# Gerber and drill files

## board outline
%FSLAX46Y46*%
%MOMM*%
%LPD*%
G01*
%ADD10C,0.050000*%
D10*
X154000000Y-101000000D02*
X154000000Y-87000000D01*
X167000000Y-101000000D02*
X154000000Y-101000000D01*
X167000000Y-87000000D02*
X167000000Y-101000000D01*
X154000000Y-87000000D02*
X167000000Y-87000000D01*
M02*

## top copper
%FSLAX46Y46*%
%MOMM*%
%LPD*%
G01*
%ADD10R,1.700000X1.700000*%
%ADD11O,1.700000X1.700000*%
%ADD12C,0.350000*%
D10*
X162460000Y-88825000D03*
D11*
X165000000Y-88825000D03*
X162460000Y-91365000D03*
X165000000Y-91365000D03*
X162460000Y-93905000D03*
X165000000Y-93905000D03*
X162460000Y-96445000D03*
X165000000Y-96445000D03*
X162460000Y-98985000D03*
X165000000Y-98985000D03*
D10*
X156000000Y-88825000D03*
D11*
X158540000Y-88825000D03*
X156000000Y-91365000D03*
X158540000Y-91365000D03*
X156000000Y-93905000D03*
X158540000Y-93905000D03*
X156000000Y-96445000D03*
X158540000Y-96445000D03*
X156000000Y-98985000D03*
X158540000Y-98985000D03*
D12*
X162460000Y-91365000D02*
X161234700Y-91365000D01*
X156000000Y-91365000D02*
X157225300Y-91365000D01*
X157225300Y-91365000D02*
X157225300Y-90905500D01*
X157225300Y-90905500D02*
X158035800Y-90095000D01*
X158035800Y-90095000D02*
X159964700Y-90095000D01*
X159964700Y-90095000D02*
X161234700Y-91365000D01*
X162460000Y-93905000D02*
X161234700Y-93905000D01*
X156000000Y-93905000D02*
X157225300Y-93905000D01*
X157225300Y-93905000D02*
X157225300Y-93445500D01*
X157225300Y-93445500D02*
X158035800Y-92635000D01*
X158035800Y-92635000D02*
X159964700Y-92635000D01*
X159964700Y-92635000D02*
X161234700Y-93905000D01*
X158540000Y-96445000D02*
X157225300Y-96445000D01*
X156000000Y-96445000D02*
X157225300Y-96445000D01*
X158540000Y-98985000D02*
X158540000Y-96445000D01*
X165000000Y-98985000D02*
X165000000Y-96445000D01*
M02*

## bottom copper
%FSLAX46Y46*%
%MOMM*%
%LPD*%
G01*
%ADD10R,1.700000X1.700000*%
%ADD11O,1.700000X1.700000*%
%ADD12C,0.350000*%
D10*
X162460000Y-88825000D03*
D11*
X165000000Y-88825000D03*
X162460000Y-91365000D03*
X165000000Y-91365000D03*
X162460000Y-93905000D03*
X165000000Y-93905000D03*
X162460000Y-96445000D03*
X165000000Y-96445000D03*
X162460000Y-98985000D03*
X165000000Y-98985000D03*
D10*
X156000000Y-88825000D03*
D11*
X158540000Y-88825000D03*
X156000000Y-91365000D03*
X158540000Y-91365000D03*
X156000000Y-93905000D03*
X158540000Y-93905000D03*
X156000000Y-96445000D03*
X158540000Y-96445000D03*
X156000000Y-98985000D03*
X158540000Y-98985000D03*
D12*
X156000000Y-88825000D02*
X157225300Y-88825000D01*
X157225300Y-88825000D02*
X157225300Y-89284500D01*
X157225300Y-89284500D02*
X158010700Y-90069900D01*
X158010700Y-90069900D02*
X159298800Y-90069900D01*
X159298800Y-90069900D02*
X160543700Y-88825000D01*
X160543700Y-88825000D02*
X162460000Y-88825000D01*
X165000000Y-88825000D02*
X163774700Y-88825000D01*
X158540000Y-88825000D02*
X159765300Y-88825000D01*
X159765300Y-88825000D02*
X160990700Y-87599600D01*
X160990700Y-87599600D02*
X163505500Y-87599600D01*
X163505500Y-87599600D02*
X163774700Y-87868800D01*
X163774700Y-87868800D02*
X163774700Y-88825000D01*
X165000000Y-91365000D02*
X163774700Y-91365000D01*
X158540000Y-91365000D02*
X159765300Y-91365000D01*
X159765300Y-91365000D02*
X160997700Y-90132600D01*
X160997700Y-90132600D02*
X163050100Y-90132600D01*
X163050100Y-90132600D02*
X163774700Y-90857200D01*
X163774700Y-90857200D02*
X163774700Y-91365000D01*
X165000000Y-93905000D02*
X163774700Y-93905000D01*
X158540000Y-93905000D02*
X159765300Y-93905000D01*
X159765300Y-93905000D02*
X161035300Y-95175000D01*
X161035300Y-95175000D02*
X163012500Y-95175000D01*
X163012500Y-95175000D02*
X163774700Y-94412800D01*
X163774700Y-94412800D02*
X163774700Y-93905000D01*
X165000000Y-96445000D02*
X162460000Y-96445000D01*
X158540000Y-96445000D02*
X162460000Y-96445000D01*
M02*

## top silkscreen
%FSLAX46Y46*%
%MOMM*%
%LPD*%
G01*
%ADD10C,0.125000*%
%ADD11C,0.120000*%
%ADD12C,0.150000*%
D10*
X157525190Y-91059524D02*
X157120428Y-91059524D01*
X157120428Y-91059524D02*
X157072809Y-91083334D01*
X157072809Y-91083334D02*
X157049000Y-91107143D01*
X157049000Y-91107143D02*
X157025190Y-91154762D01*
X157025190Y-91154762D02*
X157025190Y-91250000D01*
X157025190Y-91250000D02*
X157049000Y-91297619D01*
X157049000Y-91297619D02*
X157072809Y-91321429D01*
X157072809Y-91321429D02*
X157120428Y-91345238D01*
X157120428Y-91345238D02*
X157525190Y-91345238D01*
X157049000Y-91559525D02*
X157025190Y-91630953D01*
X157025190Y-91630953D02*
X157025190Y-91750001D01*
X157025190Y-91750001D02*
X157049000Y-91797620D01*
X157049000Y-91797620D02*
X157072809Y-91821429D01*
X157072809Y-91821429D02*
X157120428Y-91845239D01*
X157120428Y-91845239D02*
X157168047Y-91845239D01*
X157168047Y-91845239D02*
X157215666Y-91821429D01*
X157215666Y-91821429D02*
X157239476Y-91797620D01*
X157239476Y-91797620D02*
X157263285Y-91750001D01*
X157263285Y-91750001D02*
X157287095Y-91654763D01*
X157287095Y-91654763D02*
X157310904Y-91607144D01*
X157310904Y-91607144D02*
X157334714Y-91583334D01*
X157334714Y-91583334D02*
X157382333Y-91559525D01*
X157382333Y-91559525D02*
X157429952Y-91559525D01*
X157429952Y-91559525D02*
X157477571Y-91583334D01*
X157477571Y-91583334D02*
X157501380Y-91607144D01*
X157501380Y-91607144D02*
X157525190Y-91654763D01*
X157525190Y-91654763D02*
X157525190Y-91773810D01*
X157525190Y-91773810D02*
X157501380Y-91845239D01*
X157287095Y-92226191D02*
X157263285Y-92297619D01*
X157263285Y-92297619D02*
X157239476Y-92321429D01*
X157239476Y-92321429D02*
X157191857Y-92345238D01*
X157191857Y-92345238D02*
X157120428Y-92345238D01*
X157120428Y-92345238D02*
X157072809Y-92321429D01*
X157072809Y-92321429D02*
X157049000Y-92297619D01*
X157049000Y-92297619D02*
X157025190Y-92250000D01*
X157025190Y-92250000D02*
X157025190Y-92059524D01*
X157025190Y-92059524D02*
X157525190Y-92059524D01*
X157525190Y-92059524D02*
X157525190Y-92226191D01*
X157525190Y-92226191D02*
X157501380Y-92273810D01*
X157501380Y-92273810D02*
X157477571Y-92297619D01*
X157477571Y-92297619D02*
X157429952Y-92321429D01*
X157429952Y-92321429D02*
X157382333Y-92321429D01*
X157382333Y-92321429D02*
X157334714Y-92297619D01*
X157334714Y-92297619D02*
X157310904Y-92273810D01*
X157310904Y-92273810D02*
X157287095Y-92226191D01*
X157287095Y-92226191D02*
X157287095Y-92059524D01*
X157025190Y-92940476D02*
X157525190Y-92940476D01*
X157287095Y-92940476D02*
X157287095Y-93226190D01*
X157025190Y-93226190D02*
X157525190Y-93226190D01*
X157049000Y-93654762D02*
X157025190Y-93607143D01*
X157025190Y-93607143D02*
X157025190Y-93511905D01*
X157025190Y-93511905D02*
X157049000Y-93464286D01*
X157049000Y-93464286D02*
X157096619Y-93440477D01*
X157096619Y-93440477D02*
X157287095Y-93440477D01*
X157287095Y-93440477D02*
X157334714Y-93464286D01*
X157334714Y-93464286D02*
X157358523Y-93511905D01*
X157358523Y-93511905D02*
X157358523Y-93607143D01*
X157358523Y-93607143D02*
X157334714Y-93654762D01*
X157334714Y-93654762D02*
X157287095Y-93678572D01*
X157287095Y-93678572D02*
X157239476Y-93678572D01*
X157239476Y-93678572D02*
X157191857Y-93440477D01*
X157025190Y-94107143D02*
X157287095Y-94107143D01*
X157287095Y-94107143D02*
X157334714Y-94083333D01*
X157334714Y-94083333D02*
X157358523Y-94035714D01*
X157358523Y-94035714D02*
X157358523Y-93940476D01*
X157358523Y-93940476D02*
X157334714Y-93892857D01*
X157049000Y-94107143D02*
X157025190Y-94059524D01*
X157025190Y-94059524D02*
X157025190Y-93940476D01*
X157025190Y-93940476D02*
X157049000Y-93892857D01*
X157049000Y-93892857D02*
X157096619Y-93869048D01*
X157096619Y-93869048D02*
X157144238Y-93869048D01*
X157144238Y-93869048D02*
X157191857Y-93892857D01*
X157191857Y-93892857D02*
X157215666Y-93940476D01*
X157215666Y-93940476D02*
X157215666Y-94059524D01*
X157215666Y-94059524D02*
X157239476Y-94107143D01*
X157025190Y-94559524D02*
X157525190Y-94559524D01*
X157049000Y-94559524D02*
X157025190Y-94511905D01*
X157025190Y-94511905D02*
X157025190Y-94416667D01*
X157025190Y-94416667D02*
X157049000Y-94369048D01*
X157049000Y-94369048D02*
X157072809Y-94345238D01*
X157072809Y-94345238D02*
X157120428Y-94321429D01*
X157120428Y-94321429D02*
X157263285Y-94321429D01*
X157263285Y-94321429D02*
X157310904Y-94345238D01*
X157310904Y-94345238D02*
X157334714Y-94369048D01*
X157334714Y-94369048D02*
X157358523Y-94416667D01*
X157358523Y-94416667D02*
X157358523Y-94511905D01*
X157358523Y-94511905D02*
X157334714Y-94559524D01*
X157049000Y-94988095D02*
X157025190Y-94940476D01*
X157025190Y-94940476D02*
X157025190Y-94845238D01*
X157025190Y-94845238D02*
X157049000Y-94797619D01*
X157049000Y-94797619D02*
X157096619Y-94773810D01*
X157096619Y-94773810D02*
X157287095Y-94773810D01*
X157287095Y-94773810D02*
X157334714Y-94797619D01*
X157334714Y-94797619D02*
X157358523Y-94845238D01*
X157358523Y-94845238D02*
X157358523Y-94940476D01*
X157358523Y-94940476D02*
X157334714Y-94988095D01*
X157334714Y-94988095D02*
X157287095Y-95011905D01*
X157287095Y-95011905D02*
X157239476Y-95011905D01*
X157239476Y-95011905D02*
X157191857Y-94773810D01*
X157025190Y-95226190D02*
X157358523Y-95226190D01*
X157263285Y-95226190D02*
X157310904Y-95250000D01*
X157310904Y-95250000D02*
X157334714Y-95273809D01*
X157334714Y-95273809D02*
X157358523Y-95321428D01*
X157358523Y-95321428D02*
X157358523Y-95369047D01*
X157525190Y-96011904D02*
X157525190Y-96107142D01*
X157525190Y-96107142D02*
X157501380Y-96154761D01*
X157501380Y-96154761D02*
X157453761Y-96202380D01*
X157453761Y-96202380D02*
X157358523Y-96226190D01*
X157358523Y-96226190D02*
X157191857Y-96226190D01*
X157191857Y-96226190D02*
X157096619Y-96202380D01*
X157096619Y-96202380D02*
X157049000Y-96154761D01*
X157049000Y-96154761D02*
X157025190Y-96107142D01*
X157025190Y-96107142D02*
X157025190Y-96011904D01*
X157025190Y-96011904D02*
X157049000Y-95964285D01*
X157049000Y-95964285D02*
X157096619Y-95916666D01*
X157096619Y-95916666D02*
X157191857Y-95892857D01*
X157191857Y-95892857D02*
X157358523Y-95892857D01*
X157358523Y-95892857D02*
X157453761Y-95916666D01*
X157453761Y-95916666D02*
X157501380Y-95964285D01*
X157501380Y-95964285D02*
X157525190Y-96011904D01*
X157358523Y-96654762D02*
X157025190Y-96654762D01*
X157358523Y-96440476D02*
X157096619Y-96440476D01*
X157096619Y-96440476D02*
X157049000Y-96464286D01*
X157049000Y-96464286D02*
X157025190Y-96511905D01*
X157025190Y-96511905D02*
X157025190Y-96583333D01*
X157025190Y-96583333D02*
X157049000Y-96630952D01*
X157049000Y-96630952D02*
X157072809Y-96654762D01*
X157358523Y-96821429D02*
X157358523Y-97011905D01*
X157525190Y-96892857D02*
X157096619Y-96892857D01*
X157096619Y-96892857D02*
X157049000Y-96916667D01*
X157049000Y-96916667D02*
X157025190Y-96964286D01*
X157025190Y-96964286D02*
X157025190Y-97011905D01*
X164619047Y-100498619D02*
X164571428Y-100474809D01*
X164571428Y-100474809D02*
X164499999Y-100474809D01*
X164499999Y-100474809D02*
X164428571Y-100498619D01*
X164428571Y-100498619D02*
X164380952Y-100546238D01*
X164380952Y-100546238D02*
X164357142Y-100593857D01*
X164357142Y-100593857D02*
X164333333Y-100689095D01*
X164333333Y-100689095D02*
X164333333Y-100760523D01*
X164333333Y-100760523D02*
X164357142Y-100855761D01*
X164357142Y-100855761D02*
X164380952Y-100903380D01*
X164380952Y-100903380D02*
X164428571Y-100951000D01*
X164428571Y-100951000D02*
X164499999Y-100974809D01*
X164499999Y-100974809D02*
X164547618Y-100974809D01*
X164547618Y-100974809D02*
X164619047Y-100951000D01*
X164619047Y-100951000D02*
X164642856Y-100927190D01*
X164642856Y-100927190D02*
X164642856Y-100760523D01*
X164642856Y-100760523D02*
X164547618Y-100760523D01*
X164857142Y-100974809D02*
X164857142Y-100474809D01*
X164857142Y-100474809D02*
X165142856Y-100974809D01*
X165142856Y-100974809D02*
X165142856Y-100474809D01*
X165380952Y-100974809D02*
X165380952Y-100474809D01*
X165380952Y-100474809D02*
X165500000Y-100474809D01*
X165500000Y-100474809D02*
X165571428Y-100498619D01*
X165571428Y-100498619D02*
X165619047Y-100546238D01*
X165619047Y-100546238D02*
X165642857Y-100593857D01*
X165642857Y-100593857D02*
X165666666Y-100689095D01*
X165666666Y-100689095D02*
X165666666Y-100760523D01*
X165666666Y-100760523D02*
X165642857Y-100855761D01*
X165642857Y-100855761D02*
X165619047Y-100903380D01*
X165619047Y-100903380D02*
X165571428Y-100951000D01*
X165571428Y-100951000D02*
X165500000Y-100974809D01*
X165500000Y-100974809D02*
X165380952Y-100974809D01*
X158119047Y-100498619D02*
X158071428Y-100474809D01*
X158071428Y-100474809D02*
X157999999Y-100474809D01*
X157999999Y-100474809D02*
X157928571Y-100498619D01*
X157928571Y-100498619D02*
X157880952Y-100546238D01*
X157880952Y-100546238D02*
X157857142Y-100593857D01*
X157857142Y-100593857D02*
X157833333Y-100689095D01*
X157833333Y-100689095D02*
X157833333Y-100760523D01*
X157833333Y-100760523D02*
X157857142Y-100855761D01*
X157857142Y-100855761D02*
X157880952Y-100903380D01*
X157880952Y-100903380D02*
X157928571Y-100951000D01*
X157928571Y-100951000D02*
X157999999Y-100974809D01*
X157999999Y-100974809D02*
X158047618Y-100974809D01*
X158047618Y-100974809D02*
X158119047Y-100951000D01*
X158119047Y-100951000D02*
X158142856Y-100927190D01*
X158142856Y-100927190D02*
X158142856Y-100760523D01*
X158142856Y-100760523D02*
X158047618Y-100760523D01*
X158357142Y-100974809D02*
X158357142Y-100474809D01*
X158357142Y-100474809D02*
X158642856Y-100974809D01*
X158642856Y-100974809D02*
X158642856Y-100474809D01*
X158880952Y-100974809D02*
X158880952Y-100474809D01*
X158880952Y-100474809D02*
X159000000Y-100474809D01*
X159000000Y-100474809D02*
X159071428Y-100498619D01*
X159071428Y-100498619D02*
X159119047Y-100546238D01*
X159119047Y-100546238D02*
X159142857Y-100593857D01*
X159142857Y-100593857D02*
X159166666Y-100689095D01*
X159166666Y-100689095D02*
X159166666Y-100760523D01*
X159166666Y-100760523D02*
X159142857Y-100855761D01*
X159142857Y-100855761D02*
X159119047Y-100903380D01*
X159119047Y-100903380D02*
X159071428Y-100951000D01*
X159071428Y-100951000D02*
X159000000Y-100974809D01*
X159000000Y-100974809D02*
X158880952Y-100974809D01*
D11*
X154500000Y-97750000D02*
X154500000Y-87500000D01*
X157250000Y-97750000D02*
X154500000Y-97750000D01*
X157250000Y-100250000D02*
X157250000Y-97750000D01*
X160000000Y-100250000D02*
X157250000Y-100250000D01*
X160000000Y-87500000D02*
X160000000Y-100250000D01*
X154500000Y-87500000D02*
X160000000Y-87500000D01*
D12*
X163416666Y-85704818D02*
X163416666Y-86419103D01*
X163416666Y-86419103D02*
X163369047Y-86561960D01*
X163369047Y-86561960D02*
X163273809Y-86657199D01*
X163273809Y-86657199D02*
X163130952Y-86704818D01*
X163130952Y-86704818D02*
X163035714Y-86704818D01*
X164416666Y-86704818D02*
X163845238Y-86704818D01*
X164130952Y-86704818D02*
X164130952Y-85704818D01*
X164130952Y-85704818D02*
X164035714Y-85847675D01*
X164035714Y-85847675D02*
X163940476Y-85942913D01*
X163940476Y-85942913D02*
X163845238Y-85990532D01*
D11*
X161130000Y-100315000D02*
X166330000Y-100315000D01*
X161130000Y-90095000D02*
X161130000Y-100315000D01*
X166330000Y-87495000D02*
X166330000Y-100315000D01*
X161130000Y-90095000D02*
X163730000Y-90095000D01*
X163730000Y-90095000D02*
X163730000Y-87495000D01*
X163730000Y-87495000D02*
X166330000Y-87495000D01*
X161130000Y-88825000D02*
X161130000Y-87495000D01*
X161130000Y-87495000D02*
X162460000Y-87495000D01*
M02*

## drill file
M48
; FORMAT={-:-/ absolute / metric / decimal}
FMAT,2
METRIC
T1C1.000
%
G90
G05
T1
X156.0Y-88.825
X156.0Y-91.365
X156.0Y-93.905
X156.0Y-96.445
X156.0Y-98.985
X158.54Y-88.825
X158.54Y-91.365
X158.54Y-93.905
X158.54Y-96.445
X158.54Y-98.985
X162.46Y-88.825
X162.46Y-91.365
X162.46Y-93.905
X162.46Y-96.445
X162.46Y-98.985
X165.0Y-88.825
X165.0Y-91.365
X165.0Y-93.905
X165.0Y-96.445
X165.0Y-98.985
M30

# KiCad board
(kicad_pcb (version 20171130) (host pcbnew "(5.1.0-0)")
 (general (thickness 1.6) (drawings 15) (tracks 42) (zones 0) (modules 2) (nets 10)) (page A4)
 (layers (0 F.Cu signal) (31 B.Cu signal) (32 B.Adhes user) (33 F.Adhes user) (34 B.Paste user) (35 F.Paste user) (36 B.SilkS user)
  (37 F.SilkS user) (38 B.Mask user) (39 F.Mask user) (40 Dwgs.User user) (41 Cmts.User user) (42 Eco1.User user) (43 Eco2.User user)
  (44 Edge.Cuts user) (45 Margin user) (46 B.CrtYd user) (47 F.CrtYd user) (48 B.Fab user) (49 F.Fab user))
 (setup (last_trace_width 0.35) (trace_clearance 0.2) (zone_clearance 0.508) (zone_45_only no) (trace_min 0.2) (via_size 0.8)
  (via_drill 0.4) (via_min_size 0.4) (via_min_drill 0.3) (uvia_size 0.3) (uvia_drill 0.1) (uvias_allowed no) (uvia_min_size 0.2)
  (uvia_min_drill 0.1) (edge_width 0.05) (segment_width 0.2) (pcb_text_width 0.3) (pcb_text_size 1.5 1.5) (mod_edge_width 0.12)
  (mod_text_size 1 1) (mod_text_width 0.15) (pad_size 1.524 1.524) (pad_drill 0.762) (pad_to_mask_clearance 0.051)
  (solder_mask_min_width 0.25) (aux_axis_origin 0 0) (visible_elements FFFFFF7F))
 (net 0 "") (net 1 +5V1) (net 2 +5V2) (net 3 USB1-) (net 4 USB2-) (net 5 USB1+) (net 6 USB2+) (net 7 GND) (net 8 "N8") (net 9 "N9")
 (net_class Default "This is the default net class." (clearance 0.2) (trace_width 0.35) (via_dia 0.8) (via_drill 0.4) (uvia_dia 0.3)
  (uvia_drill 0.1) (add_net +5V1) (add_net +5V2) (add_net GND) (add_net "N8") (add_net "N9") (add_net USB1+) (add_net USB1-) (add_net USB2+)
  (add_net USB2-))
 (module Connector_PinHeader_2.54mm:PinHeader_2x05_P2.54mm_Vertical (layer F.Cu) (at 162.46 88.825)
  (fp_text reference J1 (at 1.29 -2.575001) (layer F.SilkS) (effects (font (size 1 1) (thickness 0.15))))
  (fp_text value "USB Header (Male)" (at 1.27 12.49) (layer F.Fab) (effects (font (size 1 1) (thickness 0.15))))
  (fp_line (start -1.33 11.49) (end 3.87 11.49) (layer F.SilkS) (width 0.12))
  (fp_line (start -1.33 1.27) (end -1.33 11.49) (layer F.SilkS) (width 0.12))
  (fp_line (start 3.87 -1.33) (end 3.87 11.49) (layer F.SilkS) (width 0.12))
  (fp_line (start -1.33 1.27) (end 1.27 1.27) (layer F.SilkS) (width 0.12))
  (fp_line (start 1.27 1.27) (end 1.27 -1.33) (layer F.SilkS) (width 0.12))
  (fp_line (start 1.27 -1.33) (end 3.87 -1.33) (layer F.SilkS) (width 0.12))
  (fp_line (start -1.33 0) (end -1.33 -1.33) (layer F.SilkS) (width 0.12))
  (fp_line (start -1.33 -1.33) (end 0 -1.33) (layer F.SilkS) (width 0.12))
  (pad 1 thru_hole rect (at 0 0) (size 1.7 1.7) (drill 1) (layers *.Cu *.Mask) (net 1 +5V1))
  (pad 2 thru_hole oval (at 2.54 0) (size 1.7 1.7) (drill 1) (layers *.Cu *.Mask) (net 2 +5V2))
  (pad 3 thru_hole oval (at 0 2.54) (size 1.7 1.7) (drill 1) (layers *.Cu *.Mask) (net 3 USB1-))
  (pad 4 thru_hole oval (at 2.54 2.54) (size 1.7 1.7) (drill 1) (layers *.Cu *.Mask) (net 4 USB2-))
  (pad 5 thru_hole oval (at 0 5.08) (size 1.7 1.7) (drill 1) (layers *.Cu *.Mask) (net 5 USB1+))
  (pad 6 thru_hole oval (at 2.54 5.08) (size 1.7 1.7) (drill 1) (layers *.Cu *.Mask) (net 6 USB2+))
  (pad 7 thru_hole oval (at 0 7.62) (size 1.7 1.7) (drill 1) (layers *.Cu *.Mask) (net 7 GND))
  (pad 8 thru_hole oval (at 2.54 7.62) (size 1.7 1.7) (drill 1) (layers *.Cu *.Mask) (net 7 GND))
  (pad 9 thru_hole oval (at 0 10.16) (size 1.7 1.7) (drill 1) (layers *.Cu *.Mask) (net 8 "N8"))
  (pad 10 thru_hole oval (at 2.54 10.16) (size 1.7 1.7) (drill 1) (layers *.Cu *.Mask) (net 7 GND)))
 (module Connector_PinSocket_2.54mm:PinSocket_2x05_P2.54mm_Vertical (layer B.Cu) (at 156 88.825 180)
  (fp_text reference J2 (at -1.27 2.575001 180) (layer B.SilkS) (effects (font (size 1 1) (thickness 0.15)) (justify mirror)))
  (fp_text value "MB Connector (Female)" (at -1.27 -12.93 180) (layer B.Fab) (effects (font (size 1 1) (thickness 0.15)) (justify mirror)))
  (pad 1 thru_hole rect (at 0 0 180) (size 1.7 1.7) (drill 1) (layers *.Cu *.Mask) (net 1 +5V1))
  (pad 2 thru_hole oval (at -2.54 0 180) (size 1.7 1.7) (drill 1) (layers *.Cu *.Mask) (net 2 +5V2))
  (pad 3 thru_hole oval (at 0 -2.54 180) (size 1.7 1.7) (drill 1) (layers *.Cu *.Mask) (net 3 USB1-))
  (pad 4 thru_hole oval (at -2.54 -2.54 180) (size 1.7 1.7) (drill 1) (layers *.Cu *.Mask) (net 4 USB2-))
  (pad 5 thru_hole oval (at 0 -5.08 180) (size 1.7 1.7) (drill 1) (layers *.Cu *.Mask) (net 5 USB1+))
  (pad 6 thru_hole oval (at -2.54 -5.08 180) (size 1.7 1.7) (drill 1) (layers *.Cu *.Mask) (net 6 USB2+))
  (pad 7 thru_hole oval (at 0 -7.62 180) (size 1.7 1.7) (drill 1) (layers *.Cu *.Mask) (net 7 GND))
  (pad 8 thru_hole oval (at -2.54 -7.62 180) (size 1.7 1.7) (drill 1) (layers *.Cu *.Mask) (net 7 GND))
  (pad 9 thru_hole oval (at 0 -10.16 180) (size 1.7 1.7) (drill 1) (layers *.Cu *.Mask) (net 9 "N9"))
  (pad 10 thru_hole oval (at -2.54 -10.16 180) (size 1.7 1.7) (drill 1) (layers *.Cu *.Mask) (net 7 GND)))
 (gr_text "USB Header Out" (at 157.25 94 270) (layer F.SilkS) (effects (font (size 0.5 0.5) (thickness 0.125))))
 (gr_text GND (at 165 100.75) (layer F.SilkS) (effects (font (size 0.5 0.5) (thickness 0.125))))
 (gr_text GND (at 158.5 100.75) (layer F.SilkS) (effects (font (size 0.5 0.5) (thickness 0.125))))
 (gr_line (start 154.5 97.75) (end 154.5 87.5) (layer F.SilkS) (width 0.12))
 (gr_line (start 157.25 97.75) (end 154.5 97.75) (layer F.SilkS) (width 0.12))
 (gr_line (start 157.25 100.25) (end 157.25 97.75) (layer F.SilkS) (width 0.12))
 (gr_line (start 160 100.25) (end 157.25 100.25) (layer F.SilkS) (width 0.12))
 (gr_line (start 160 87.5) (end 160 100.25) (layer F.SilkS) (width 0.12))
 (gr_line (start 154.5 87.5) (end 160 87.5) (layer F.SilkS) (width 0.12))
 (gr_line (start 154 101) (end 154 87) (layer Edge.Cuts) (width 0.05))
 (gr_line (start 167 101) (end 154 101) (layer Edge.Cuts) (width 0.05))
 (gr_line (start 167 87) (end 167 101) (layer Edge.Cuts) (width 0.05))
 (gr_line (start 154 87) (end 167 87) (layer Edge.Cuts) (width 0.05))
 (segment (start 156 88.825) (end 157.2253 88.825) (width 0.35) (layer B.Cu) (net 1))
 (segment (start 157.2253 88.825) (end 157.2253 89.2845) (width 0.35) (layer B.Cu) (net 1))
 (segment (start 157.2253 89.2845) (end 158.0107 90.0699) (width 0.35) (layer B.Cu) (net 1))
 (segment (start 158.0107 90.0699) (end 159.2988 90.0699) (width 0.35) (layer B.Cu) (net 1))
 (segment (start 159.2988 90.0699) (end 160.5437 88.825) (width 0.35) (layer B.Cu) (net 1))
 (segment (start 160.5437 88.825) (end 162.46 88.825) (width 0.35) (layer B.Cu) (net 1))
 (segment (start 165 88.825) (end 163.7747 88.825) (width 0.35) (layer B.Cu) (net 2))
 (segment (start 158.54 88.825) (end 159.7653 88.825) (width 0.35) (layer B.Cu) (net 2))
 (segment (start 159.7653 88.825) (end 160.9907 87.5996) (width 0.35) (layer B.Cu) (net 2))
 (segment (start 160.9907 87.5996) (end 163.5055 87.5996) (width 0.35) (layer B.Cu) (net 2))
 (segment (start 163.5055 87.5996) (end 163.7747 87.8688) (width 0.35) (layer B.Cu) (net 2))
 (segment (start 163.7747 87.8688) (end 163.7747 88.825) (width 0.35) (layer B.Cu) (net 2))
 (segment (start 162.46 91.365) (end 161.2347 91.365) (width 0.35) (layer F.Cu) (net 3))
 (segment (start 156 91.365) (end 157.2253 91.365) (width 0.35) (layer F.Cu) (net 3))
 (segment (start 157.2253 91.365) (end 157.2253 90.9055) (width 0.35) (layer F.Cu) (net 3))
 (segment (start 157.2253 90.9055) (end 158.0358 90.095) (width 0.35) (layer F.Cu) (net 3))
 (segment (start 158.0358 90.095) (end 159.9647 90.095) (width 0.35) (layer F.Cu) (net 3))
 (segment (start 159.9647 90.095) (end 161.2347 91.365) (width 0.35) (layer F.Cu) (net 3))
 (segment (start 165 91.365) (end 163.7747 91.365) (width 0.35) (layer B.Cu) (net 4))
 (segment (start 158.54 91.365) (end 159.7653 91.365) (width 0.35) (layer B.Cu) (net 4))
 (segment (start 159.7653 91.365) (end 160.9977 90.1326) (width 0.35) (layer B.Cu) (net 4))
 (segment (start 160.9977 90.1326) (end 163.0501 90.1326) (width 0.35) (layer B.Cu) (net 4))
 (segment (start 163.0501 90.1326) (end 163.7747 90.8572) (width 0.35) (layer B.Cu) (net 4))
 (segment (start 163.7747 90.8572) (end 163.7747 91.365) (width 0.35) (layer B.Cu) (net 4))
 (segment (start 162.46 93.905) (end 161.2347 93.905) (width 0.35) (layer F.Cu) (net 5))
 (segment (start 156 93.905) (end 157.2253 93.905) (width 0.35) (layer F.Cu) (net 5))
 (segment (start 157.2253 93.905) (end 157.2253 93.4455) (width 0.35) (layer F.Cu) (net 5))
 (segment (start 157.2253 93.4455) (end 158.0358 92.635) (width 0.35) (layer F.Cu) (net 5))
 (segment (start 158.0358 92.635) (end 159.9647 92.635) (width 0.35) (layer F.Cu) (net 5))
 (segment (start 159.9647 92.635) (end 161.2347 93.905) (width 0.35) (layer F.Cu) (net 5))
 (segment (start 165 93.905) (end 163.7747 93.905) (width 0.35) (layer B.Cu) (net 6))
 (segment (start 158.54 93.905) (end 159.7653 93.905) (width 0.35) (layer B.Cu) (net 6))
 (segment (start 159.7653 93.905) (end 161.0353 95.175) (width 0.35) (layer B.Cu) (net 6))
 (segment (start 161.0353 95.175) (end 163.0125 95.175) (width 0.35) (layer B.Cu) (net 6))
 (segment (start 163.0125 95.175) (end 163.7747 94.4128) (width 0.35) (layer B.Cu) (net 6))
 (segment (start 163.7747 94.4128) (end 163.7747 93.905) (width 0.35) (layer B.Cu) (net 6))
 (segment (start 158.54 96.445) (end 157.2253 96.445) (width 0.35) (layer F.Cu) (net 7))
 (segment (start 156 96.445) (end 157.2253 96.445) (width 0.35) (layer F.Cu) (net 7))
 (segment (start 158.54 98.985) (end 158.54 96.445) (width 0.35) (layer F.Cu) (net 7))
 (segment (start 165 96.445) (end 162.46 96.445) (width 0.35) (layer B.Cu) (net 7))
 (segment (start 165 98.985) (end 165 96.445) (width 0.35) (layer F.Cu) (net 7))
 (segment (start 158.54 96.445) (end 162.46 96.445) (width 0.35) (layer B.Cu) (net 7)))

